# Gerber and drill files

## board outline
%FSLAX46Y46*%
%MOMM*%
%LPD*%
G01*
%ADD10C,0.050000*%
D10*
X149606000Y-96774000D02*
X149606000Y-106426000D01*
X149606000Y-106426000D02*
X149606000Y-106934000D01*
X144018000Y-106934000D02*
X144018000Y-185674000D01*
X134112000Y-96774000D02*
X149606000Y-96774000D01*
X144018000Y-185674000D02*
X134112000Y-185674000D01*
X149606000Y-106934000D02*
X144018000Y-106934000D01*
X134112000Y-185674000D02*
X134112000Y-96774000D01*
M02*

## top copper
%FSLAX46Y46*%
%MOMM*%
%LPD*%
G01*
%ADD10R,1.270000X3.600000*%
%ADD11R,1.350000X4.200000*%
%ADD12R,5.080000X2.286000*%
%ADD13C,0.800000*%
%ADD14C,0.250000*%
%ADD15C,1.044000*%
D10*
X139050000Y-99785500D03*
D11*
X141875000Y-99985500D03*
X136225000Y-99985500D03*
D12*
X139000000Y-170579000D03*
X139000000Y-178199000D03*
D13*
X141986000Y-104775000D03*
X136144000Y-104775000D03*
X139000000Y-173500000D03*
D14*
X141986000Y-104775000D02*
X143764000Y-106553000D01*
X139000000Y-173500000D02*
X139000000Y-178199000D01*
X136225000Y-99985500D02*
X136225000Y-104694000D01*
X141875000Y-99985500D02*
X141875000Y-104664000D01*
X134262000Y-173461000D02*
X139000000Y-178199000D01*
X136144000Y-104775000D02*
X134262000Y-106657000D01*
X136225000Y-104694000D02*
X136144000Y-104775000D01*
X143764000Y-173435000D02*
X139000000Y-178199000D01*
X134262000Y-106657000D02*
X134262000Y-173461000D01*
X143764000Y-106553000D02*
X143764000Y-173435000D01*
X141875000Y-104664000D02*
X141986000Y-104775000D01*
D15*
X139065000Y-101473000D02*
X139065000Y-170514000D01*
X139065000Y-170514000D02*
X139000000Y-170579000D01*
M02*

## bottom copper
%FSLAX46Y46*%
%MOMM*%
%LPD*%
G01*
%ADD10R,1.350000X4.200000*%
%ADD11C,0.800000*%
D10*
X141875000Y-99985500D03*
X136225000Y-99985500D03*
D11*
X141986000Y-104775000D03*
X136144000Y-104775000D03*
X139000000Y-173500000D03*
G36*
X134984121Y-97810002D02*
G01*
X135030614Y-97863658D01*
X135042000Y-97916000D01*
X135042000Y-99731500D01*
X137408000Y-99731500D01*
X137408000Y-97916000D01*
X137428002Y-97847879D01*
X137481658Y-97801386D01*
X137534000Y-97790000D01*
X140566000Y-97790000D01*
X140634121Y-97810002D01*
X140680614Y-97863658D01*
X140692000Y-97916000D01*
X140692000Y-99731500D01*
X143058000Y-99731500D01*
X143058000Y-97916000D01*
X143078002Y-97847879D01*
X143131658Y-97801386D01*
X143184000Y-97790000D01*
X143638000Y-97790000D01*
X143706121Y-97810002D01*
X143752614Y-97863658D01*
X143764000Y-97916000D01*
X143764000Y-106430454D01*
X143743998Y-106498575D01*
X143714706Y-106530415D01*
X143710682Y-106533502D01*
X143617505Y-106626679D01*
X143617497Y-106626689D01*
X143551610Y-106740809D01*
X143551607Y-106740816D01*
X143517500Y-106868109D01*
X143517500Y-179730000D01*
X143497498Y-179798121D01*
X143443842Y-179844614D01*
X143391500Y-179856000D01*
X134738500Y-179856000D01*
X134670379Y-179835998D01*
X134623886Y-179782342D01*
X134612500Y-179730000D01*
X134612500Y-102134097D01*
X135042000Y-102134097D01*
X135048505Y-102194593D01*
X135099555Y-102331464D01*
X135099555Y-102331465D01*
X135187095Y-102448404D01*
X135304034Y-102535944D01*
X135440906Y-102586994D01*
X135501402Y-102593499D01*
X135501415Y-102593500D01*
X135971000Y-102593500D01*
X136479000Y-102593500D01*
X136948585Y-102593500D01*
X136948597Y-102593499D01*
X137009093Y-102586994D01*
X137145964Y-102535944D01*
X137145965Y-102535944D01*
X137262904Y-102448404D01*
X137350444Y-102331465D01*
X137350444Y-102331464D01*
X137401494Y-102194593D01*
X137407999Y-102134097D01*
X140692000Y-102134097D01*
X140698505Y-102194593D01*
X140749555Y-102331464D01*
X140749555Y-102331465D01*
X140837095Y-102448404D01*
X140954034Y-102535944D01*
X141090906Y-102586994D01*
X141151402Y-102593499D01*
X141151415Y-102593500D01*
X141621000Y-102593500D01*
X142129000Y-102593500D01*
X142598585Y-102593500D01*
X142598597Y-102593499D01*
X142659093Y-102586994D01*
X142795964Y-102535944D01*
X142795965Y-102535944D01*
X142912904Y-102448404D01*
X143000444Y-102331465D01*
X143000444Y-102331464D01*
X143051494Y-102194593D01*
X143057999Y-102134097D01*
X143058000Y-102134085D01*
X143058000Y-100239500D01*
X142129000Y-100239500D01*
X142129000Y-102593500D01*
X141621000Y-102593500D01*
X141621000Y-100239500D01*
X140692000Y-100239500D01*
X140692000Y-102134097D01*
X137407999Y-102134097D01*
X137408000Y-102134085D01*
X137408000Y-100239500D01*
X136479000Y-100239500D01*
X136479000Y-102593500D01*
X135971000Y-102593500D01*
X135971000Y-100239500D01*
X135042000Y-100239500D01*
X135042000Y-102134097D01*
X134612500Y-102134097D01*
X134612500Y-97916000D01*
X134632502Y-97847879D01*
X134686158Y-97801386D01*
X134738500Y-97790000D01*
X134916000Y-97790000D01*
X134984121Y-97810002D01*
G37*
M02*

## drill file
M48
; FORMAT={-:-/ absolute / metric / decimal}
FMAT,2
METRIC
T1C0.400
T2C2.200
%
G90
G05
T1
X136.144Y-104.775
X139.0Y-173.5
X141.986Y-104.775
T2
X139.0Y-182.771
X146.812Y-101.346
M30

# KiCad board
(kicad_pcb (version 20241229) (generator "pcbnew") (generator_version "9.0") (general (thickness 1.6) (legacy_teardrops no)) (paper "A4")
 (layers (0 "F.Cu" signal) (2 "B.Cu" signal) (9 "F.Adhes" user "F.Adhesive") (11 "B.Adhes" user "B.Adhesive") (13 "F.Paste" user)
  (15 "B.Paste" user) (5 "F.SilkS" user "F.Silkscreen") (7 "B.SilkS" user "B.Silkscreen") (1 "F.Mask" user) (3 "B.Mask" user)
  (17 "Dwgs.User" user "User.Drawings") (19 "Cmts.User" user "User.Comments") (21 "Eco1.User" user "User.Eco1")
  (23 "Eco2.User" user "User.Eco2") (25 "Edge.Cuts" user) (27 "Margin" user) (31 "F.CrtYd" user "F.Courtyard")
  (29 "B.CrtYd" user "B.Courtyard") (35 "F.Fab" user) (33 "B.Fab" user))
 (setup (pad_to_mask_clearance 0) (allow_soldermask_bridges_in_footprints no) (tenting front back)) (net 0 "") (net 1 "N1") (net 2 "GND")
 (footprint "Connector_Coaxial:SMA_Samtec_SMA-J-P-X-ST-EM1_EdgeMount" (layer "F.Cu") (at 139.05 99.9855 180)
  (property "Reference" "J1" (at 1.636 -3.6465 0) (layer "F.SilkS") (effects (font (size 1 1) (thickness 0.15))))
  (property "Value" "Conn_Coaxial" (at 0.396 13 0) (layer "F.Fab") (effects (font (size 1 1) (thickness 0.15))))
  (pad "1" smd rect (at 0 0.2 180) (size 1.27 3.6) (layers "F.Cu" "F.Mask" "F.Paste") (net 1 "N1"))
  (pad "2" smd rect (at -2.825 0 180) (size 1.35 4.2) (layers "F.Cu" "F.Mask" "F.Paste") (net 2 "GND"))
  (pad "2" smd rect (at -2.825 0 180) (size 1.35 4.2) (layers "B.Cu" "B.Mask" "B.Paste") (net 2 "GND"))
  (pad "2" smd rect (at 2.825 0 180) (size 1.35 4.2) (layers "F.Cu" "F.Mask" "F.Paste") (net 2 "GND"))
  (pad "2" smd rect (at 2.825 0 180) (size 1.35 4.2) (layers "B.Cu" "B.Mask" "B.Paste") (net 2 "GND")))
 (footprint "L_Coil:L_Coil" (layer "F.Cu") (at 139 171.595 180)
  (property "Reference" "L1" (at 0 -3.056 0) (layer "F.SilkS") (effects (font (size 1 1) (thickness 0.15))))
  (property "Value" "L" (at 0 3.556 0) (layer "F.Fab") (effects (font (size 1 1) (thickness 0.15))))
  (pad "1" smd rect (at 0 1.016 180) (size 5.08 2.286) (layers "F.Cu" "F.Mask" "F.Paste") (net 1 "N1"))
  (pad "2" smd rect (at 0 -6.604 180) (size 5.08 2.286) (layers "F.Cu" "F.Mask" "F.Paste") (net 2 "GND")))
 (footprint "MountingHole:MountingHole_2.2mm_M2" (layer "F.Cu") (at 139 182.771)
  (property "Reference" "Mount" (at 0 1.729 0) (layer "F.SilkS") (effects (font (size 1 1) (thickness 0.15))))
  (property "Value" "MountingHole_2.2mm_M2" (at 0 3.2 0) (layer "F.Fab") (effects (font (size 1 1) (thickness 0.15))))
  (pad "" np_thru_hole circle (at 0 0) (size 2.2 2.2) (drill 2.2) (layers "*.Cu" "*.Mask")))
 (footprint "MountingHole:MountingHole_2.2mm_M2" (layer "F.Cu") (at 146.812 101.346)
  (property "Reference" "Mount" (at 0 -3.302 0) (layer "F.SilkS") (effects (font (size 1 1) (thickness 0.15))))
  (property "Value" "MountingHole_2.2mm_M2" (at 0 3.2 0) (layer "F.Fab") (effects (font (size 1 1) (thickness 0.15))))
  (pad "" np_thru_hole circle (at 0 0) (size 2.2 2.2) (drill 2.2) (layers "*.Cu" "*.Mask")))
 (gr_line (start 149.606 96.774) (end 149.606 106.426) (stroke (width 0.05) (type solid)) (layer "Edge.Cuts"))
 (gr_line (start 149.606 106.426) (end 149.606 106.934) (stroke (width 0.05) (type solid)) (layer "Edge.Cuts"))
 (gr_line (start 144.018 106.934) (end 144.018 185.674) (stroke (width 0.05) (type solid)) (layer "Edge.Cuts"))
 (gr_line (start 134.112 96.774) (end 149.606 96.774) (stroke (width 0.05) (type solid)) (layer "Edge.Cuts"))
 (gr_line (start 144.018 185.674) (end 134.112 185.674) (stroke (width 0.05) (type solid)) (layer "Edge.Cuts"))
 (gr_line (start 149.606 106.934) (end 144.018 106.934) (stroke (width 0.05) (type solid)) (layer "Edge.Cuts"))
 (gr_line (start 134.112 185.674) (end 134.112 96.774) (stroke (width 0.05) (type solid)) (layer "Edge.Cuts"))
 (segment (start 141.986 104.775) (end 143.764 106.553) (width 0.25) (layer "F.Cu") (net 2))
 (segment (start 139 173.5) (end 139 178.199) (width 0.25) (layer "F.Cu") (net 2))
 (segment (start 136.225 99.9855) (end 136.225 104.694) (width 0.25) (layer "F.Cu") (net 2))
 (segment (start 141.875 99.9855) (end 141.875 104.664) (width 0.25) (layer "F.Cu") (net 2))
 (segment (start 134.262 173.461) (end 139 178.199) (width 0.25) (layer "F.Cu") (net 2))
 (segment (start 136.144 104.775) (end 134.262 106.657) (width 0.25) (layer "F.Cu") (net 2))
 (segment (start 136.225 104.694) (end 136.144 104.775) (width 0.25) (layer "F.Cu") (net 2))
 (segment (start 143.764 173.435) (end 139 178.199) (width 0.25) (layer "F.Cu") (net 2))
 (segment (start 134.262 106.657) (end 134.262 173.461) (width 0.25) (layer "F.Cu") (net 2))
 (segment (start 143.764 106.553) (end 143.764 173.435) (width 0.25) (layer "F.Cu") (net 2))
 (segment (start 141.875 104.664) (end 141.986 104.775) (width 0.25) (layer "F.Cu") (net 2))
 (via (at 141.986 104.775) (size 0.8) (drill 0.4) (layers "F.Cu" "B.Cu") (free yes) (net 2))
 (via (at 136.144 104.775) (size 0.8) (drill 0.4) (layers "F.Cu" "B.Cu") (free yes) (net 2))
 (via (at 139 173.5) (size 0.8) (drill 0.4) (layers "F.Cu" "B.Cu") (free yes) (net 2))
 (segment (start 139.065 101.473) (end 139.065 170.514) (width 1.044) (layer "F.Cu") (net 1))
 (segment (start 139.065 170.514) (end 139 170.579) (width 1.044) (layer "F.Cu") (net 1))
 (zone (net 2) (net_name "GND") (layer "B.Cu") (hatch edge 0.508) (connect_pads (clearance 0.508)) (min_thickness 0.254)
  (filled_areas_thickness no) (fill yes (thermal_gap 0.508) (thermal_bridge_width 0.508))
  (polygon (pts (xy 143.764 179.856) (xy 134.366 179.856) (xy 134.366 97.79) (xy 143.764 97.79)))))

